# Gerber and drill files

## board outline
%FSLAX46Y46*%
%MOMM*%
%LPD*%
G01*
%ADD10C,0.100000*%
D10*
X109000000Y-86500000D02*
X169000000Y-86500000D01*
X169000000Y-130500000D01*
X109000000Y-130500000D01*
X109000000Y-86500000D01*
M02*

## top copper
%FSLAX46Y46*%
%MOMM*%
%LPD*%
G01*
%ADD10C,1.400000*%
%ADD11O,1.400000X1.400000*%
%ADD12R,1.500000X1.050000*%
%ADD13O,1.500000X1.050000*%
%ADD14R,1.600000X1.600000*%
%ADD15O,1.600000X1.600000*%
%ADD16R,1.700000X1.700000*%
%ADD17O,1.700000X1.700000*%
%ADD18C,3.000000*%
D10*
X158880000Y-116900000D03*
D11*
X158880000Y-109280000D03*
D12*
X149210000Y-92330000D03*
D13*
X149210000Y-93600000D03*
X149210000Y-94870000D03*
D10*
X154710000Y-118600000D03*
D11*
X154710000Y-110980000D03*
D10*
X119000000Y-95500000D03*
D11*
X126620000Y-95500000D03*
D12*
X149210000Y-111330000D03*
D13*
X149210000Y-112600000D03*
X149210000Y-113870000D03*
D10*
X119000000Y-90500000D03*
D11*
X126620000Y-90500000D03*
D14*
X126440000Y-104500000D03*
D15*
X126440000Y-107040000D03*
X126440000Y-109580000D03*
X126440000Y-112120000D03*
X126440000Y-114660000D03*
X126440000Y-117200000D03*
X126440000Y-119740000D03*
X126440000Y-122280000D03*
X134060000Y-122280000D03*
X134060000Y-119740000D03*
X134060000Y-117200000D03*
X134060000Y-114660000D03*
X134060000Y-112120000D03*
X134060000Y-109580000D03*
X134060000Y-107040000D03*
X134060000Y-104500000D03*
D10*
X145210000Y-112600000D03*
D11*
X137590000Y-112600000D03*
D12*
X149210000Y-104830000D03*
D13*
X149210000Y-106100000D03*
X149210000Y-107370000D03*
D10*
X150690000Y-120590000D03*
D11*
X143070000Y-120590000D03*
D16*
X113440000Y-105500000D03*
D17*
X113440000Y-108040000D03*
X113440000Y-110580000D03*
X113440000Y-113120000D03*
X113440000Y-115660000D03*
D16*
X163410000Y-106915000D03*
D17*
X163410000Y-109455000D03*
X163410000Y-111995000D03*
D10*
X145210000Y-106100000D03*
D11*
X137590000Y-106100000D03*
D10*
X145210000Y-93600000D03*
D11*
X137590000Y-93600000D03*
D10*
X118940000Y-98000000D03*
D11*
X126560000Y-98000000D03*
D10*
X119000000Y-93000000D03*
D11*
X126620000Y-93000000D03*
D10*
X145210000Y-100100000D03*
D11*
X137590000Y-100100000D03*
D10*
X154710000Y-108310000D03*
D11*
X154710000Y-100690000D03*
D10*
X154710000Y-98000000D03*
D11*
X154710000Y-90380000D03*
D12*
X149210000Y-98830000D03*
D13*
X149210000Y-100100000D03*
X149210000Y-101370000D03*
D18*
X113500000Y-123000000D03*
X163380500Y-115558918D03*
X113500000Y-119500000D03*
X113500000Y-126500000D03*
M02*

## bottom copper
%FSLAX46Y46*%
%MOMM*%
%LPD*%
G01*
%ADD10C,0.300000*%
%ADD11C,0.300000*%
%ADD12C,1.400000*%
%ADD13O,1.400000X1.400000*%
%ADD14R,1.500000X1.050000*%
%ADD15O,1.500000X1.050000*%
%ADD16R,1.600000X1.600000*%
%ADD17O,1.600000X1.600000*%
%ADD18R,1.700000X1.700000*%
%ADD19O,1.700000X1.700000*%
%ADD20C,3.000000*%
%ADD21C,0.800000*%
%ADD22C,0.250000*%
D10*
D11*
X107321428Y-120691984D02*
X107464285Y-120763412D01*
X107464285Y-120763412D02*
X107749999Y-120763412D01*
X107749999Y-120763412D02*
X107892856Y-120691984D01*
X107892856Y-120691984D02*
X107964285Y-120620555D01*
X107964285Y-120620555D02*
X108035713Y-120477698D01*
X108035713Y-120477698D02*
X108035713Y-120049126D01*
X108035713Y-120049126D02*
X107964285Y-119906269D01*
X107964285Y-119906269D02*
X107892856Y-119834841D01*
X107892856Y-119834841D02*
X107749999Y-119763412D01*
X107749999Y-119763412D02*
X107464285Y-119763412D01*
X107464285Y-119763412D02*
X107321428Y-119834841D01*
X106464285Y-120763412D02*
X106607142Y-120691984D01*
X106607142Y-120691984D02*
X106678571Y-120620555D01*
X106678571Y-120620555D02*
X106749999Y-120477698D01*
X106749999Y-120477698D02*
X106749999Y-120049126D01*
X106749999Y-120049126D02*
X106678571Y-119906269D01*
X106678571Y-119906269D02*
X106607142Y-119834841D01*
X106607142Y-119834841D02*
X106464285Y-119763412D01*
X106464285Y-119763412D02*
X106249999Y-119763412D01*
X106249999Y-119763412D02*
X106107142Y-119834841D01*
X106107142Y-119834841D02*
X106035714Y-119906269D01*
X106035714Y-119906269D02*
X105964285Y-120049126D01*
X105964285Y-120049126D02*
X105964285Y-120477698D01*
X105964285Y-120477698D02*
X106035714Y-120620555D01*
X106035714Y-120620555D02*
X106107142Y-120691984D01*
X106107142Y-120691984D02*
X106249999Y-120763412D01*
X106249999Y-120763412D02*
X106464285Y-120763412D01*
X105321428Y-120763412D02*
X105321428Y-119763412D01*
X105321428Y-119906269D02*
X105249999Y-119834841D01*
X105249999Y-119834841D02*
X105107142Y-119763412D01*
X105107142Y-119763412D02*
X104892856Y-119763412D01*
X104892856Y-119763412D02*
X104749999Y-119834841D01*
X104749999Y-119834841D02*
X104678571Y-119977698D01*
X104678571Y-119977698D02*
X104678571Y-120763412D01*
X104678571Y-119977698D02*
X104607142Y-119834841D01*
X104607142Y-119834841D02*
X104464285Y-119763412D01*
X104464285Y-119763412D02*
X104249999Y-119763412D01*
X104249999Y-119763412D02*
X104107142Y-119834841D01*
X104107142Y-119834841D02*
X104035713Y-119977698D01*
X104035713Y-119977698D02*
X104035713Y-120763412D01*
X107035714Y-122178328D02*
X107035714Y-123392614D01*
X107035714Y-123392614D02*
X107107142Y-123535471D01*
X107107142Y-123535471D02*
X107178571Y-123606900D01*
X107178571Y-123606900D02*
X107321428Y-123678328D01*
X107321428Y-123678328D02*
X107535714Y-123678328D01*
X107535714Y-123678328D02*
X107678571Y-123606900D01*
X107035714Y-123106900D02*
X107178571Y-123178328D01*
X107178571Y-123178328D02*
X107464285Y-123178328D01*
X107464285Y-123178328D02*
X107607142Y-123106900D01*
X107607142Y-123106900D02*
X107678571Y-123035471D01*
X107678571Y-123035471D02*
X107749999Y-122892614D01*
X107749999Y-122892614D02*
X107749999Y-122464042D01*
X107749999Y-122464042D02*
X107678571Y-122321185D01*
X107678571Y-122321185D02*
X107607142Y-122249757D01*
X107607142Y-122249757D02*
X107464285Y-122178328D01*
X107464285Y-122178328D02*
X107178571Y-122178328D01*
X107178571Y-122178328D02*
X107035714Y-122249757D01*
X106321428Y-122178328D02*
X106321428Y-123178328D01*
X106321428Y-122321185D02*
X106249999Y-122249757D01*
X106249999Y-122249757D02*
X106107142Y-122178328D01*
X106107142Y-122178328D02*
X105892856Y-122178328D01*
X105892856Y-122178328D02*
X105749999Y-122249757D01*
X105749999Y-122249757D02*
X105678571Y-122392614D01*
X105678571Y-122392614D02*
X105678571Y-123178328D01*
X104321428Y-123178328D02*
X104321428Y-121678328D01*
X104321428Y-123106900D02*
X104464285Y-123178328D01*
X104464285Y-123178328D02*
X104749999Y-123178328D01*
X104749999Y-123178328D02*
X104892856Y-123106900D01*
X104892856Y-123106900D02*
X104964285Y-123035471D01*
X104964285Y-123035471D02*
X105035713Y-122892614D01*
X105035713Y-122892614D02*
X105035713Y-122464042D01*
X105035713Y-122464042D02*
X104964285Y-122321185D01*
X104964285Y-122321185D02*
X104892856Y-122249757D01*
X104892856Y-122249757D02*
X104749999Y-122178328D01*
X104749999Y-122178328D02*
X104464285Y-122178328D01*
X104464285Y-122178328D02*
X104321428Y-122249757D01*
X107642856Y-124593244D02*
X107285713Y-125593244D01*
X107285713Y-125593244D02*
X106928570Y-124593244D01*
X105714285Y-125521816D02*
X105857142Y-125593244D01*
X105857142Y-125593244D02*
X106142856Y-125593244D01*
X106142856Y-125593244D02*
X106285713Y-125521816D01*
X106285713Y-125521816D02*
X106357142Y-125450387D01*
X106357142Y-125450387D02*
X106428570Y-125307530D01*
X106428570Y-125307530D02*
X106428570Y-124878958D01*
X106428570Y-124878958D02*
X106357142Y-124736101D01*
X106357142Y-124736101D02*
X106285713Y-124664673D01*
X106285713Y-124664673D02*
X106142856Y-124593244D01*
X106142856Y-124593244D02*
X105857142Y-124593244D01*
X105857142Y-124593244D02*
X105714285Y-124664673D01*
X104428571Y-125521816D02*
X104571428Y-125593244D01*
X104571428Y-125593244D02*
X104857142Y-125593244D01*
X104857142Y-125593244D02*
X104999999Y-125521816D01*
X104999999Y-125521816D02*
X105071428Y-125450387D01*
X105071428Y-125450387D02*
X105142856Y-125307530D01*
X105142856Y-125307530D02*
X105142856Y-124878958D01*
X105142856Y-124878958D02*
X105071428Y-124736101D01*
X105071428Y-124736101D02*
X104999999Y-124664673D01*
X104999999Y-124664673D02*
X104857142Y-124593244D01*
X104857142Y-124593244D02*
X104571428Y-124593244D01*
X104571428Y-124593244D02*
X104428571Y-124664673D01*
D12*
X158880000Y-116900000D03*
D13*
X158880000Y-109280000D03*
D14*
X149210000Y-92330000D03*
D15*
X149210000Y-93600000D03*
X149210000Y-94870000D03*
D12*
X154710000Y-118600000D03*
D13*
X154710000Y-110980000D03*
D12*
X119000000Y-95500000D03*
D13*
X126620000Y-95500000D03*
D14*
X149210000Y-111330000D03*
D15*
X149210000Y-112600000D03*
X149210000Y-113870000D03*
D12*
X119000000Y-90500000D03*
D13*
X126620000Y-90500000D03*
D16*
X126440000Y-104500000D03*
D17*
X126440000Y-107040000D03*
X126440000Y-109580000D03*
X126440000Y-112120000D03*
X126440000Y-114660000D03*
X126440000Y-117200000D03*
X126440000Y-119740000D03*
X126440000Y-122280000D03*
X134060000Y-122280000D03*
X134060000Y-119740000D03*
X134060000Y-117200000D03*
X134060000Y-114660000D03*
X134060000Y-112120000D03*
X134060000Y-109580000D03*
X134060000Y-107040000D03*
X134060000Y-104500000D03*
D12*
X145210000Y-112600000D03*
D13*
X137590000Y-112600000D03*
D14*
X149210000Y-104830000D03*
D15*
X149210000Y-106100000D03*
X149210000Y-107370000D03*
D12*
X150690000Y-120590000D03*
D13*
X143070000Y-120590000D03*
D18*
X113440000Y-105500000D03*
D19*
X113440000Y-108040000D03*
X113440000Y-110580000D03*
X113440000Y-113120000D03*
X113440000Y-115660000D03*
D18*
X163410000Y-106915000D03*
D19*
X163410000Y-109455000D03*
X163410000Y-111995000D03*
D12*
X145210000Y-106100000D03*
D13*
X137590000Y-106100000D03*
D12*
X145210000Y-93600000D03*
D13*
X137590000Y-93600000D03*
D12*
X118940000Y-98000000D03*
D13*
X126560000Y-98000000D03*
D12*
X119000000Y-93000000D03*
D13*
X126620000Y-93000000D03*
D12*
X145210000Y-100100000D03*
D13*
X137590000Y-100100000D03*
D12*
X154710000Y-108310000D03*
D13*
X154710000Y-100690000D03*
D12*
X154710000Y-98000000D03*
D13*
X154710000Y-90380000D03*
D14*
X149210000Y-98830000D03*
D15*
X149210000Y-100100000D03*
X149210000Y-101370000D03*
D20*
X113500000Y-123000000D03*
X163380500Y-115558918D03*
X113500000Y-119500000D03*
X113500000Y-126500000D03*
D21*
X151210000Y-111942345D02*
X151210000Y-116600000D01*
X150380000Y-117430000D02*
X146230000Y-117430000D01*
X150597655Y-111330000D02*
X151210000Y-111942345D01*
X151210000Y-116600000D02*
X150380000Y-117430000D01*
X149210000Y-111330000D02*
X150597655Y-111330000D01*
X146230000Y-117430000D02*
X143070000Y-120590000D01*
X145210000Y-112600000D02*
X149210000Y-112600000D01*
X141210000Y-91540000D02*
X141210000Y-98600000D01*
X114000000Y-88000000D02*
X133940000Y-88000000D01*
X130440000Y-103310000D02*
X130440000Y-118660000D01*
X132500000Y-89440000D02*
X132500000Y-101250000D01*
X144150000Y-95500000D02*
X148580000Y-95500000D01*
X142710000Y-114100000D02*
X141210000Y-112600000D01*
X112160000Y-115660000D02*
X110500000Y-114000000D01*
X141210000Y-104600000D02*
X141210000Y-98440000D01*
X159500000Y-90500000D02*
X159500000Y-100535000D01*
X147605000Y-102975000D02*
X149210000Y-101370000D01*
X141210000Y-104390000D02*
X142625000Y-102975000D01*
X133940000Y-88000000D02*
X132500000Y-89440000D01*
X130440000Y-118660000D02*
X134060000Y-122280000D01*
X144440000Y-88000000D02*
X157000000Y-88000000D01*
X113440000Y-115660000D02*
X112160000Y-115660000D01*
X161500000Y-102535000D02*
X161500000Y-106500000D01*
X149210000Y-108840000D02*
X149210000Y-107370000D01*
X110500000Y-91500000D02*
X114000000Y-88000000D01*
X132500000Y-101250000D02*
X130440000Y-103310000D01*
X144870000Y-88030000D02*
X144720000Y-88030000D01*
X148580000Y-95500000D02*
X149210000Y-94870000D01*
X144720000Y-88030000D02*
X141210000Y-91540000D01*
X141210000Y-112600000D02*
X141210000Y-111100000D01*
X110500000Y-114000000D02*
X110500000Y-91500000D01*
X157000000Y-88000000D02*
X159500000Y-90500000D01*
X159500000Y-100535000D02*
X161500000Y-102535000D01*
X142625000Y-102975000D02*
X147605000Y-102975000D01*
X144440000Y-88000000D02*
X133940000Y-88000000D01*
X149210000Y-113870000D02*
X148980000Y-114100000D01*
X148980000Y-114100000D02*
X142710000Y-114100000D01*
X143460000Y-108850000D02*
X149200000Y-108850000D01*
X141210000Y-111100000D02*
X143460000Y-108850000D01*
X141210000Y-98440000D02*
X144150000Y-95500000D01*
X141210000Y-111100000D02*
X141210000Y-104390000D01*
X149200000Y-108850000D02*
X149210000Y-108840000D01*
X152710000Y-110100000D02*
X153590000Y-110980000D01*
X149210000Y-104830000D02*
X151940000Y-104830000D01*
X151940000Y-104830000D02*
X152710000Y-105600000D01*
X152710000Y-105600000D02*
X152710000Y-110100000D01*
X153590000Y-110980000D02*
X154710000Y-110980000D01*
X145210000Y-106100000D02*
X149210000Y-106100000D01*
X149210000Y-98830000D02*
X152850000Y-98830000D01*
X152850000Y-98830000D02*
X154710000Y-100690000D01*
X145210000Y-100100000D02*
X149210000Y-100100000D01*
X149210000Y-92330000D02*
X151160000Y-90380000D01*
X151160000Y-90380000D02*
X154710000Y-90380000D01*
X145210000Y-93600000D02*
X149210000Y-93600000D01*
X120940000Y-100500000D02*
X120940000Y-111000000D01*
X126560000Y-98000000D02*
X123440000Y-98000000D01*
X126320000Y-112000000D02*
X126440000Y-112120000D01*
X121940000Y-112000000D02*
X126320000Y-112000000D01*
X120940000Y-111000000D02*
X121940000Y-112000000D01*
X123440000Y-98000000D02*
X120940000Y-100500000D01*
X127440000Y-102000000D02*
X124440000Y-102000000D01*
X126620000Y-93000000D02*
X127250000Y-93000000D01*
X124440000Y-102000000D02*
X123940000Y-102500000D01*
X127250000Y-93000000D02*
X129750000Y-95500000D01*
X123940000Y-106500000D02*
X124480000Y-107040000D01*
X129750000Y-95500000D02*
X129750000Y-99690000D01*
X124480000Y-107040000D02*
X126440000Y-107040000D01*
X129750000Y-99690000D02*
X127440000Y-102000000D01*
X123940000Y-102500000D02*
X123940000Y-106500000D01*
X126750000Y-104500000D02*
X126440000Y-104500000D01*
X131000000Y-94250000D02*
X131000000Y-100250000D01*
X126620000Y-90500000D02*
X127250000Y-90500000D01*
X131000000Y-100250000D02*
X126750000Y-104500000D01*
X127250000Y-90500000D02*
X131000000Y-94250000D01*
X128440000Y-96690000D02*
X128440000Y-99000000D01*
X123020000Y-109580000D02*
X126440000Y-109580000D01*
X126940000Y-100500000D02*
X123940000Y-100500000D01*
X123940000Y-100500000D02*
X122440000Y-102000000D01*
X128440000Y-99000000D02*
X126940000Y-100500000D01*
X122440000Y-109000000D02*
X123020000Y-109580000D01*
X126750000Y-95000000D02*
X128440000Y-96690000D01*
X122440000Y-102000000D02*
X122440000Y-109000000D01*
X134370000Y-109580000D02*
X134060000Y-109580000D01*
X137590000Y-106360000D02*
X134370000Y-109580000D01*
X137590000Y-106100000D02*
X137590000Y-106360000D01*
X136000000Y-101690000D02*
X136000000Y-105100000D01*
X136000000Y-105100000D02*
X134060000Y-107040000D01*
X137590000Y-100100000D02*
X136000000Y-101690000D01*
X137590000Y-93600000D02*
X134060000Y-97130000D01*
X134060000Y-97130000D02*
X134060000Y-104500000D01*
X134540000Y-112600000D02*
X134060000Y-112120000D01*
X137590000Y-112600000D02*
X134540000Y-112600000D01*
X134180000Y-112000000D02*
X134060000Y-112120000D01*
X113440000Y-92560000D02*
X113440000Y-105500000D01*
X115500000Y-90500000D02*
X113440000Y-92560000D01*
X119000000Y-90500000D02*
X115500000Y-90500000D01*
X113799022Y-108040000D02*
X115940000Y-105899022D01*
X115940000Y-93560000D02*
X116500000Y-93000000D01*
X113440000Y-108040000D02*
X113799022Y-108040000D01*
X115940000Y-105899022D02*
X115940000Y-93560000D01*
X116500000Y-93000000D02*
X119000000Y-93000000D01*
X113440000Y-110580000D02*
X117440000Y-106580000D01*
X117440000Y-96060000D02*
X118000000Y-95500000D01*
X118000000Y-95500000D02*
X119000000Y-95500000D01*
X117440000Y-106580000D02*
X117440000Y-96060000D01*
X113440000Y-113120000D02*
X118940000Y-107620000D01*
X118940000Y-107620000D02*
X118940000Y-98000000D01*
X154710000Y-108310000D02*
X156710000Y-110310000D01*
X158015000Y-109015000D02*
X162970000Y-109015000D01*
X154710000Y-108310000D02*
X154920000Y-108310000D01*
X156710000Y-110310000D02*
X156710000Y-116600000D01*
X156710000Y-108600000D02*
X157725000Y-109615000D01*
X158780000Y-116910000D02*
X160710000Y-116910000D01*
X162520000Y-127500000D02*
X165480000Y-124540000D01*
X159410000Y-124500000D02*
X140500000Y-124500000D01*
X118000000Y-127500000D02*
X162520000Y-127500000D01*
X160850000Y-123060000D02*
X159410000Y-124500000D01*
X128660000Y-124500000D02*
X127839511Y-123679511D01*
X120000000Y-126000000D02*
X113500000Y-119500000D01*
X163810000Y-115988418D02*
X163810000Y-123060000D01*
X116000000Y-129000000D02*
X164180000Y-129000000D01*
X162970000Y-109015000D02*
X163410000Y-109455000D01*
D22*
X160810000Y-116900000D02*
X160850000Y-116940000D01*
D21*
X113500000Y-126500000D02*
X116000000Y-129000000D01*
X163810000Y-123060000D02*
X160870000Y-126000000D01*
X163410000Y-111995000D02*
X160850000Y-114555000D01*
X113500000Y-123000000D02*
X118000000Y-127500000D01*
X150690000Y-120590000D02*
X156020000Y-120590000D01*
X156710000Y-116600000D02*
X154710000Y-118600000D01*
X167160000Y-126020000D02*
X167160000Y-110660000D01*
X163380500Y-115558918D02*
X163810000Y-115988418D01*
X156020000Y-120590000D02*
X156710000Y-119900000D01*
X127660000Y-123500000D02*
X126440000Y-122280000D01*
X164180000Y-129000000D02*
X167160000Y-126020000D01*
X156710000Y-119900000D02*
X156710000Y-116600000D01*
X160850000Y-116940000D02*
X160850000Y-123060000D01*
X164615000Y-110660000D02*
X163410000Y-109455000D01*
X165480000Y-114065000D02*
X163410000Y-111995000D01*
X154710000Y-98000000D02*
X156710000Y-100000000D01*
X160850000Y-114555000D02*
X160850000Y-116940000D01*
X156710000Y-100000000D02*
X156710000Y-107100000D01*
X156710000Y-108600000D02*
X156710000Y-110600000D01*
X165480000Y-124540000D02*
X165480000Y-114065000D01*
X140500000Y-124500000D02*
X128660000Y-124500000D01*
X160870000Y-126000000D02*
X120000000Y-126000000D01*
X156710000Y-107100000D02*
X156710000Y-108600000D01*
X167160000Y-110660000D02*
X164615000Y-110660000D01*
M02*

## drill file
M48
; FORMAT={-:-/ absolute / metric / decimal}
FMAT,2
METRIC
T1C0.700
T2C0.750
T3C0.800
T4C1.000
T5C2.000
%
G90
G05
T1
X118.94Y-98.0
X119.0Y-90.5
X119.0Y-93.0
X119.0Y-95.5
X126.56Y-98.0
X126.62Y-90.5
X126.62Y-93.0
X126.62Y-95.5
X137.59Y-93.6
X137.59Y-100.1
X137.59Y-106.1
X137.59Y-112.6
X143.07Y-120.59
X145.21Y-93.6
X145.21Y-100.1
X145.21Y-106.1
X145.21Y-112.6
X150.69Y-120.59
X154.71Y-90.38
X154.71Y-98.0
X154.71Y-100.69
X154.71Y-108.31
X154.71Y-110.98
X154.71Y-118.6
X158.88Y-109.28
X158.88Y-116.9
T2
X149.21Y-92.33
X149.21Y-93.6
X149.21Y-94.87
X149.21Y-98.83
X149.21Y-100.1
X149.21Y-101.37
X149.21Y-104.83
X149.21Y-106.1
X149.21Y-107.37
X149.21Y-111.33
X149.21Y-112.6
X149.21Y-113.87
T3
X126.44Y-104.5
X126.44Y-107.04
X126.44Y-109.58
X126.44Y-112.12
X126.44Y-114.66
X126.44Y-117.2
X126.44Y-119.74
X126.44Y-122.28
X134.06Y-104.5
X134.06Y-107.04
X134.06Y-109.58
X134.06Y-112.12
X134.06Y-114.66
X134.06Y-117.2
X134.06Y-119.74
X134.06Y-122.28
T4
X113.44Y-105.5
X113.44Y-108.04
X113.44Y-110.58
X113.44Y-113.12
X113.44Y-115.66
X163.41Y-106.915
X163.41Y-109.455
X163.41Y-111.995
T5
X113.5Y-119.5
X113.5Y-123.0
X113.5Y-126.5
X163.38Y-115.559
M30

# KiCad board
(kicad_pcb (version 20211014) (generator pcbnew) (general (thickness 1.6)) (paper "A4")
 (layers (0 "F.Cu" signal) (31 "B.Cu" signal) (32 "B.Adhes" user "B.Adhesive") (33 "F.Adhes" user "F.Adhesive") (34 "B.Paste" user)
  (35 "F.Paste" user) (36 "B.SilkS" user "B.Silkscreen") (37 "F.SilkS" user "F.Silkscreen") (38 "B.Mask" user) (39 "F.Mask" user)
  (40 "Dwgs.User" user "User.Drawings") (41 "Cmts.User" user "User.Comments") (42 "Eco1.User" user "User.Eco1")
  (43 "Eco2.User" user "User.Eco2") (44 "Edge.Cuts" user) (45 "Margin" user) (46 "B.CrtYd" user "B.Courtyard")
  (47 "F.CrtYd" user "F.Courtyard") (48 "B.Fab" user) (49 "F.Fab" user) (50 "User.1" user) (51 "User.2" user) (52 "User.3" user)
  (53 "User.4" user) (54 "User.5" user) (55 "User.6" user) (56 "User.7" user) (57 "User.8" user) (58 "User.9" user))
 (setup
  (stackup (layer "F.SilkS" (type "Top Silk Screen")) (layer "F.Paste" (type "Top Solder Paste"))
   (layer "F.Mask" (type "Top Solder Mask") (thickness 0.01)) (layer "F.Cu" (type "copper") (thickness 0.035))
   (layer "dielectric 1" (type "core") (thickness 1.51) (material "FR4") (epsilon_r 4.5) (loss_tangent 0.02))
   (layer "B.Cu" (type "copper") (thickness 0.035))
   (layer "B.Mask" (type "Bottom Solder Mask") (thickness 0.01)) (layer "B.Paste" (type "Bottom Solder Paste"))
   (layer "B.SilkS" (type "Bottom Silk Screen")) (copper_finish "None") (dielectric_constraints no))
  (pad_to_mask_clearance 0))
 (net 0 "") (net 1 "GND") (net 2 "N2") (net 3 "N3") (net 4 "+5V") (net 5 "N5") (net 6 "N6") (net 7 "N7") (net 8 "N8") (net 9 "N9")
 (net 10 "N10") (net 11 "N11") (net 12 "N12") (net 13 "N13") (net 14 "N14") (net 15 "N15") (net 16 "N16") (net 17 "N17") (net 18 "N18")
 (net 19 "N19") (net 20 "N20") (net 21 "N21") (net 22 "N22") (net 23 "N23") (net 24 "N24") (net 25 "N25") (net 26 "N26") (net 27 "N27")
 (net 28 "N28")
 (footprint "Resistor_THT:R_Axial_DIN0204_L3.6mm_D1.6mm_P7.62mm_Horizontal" (layer "F.Cu") (at 158.88 116.9 90)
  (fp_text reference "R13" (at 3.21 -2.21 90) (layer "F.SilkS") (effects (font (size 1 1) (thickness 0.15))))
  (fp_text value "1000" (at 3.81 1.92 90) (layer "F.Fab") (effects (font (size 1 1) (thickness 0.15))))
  (pad "1" thru_hole circle (at 0 0 90) (size 1.4 1.4) (drill 0.7) (layers *.Cu *.Mask) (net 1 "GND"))
  (pad "2" thru_hole oval (at 7.62 0 90) (size 1.4 1.4) (drill 0.7) (layers *.Cu *.Mask) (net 1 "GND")))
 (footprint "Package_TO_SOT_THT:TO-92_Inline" (layer "F.Cu") (at 149.21 92.33 -90)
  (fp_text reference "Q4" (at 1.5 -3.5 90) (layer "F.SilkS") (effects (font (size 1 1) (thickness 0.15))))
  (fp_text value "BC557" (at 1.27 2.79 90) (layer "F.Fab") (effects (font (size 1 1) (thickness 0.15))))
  (pad "1" thru_hole rect (at 0 0 270) (size 1.05 1.5) (drill 0.75) (layers *.Cu *.Mask) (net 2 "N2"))
  (pad "2" thru_hole oval (at 1.27 0 270) (size 1.05 1.5) (drill 0.75) (layers *.Cu *.Mask) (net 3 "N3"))
  (pad "3" thru_hole oval (at 2.54 0 270) (size 1.05 1.5) (drill 0.75) (layers *.Cu *.Mask) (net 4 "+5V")))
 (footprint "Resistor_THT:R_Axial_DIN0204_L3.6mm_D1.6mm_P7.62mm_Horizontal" (layer "F.Cu") (at 154.71 118.6 90)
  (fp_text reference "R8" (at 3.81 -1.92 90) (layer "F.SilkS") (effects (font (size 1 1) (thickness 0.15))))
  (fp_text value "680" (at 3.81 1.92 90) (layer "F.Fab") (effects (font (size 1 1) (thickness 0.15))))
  (pad "1" thru_hole circle (at 0 0 90) (size 1.4 1.4) (drill 0.7) (layers *.Cu *.Mask) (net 1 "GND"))
  (pad "2" thru_hole oval (at 7.62 0 90) (size 1.4 1.4) (drill 0.7) (layers *.Cu *.Mask) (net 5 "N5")))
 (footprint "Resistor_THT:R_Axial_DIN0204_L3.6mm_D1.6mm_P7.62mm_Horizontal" (layer "F.Cu") (at 119 95.5)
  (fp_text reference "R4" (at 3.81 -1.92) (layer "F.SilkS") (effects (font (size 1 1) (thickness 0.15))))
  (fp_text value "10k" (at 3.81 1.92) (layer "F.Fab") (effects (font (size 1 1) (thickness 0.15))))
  (pad "1" thru_hole circle (at 0 0) (size 1.4 1.4) (drill 0.7) (layers *.Cu *.Mask) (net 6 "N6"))
  (pad "2" thru_hole oval (at 7.62 0) (size 1.4 1.4) (drill 0.7) (layers *.Cu *.Mask) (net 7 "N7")))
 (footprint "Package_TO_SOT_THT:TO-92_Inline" (layer "F.Cu") (at 149.21 111.33 -90)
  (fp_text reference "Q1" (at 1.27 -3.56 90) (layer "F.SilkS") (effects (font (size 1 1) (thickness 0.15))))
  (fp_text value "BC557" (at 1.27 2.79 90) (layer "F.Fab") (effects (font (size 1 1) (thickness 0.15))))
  (pad "1" thru_hole rect (at 0 0 270) (size 1.05 1.5) (drill 0.75) (layers *.Cu *.Mask) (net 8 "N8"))
  (pad "2" thru_hole oval (at 1.27 0 270) (size 1.05 1.5) (drill 0.75) (layers *.Cu *.Mask) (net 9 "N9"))
  (pad "3" thru_hole oval (at 2.54 0 270) (size 1.05 1.5) (drill 0.75) (layers *.Cu *.Mask) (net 4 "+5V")))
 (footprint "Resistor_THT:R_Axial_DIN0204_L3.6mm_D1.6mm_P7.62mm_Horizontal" (layer "F.Cu") (at 119 90.5)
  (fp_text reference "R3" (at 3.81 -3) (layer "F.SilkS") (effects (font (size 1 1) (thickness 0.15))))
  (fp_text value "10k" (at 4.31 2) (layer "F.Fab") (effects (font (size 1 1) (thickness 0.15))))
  (pad "1" thru_hole circle (at 0 0) (size 1.4 1.4) (drill 0.7) (layers *.Cu *.Mask) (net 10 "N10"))
  (pad "2" thru_hole oval (at 7.62 0) (size 1.4 1.4) (drill 0.7) (layers *.Cu *.Mask) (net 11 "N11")))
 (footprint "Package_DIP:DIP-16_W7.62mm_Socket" (layer "F.Cu") (at 126.44 104.5)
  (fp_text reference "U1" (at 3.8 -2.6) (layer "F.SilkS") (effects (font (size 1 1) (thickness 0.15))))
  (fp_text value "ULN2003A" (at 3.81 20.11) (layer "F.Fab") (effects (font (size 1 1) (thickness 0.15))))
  (pad "1" thru_hole rect (at 0 0) (size 1.6 1.6) (drill 0.8) (layers *.Cu *.Mask) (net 11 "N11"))
  (pad "2" thru_hole oval (at 0 2.54) (size 1.6 1.6) (drill 0.8) (layers *.Cu *.Mask) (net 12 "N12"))
  (pad "3" thru_hole oval (at 0 5.08) (size 1.6 1.6) (drill 0.8) (layers *.Cu *.Mask) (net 7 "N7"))
  (pad "4" thru_hole oval (at 0 7.62) (size 1.6 1.6) (drill 0.8) (layers *.Cu *.Mask) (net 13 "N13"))
  (pad "5" thru_hole oval (at 0 10.16) (size 1.6 1.6) (drill 0.8) (layers *.Cu *.Mask) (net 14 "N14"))
  (pad "6" thru_hole oval (at 0 12.7) (size 1.6 1.6) (drill 0.8) (layers *.Cu *.Mask) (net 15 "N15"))
  (pad "7" thru_hole oval (at 0 15.24) (size 1.6 1.6) (drill 0.8) (layers *.Cu *.Mask) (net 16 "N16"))
  (pad "8" thru_hole oval (at 0 17.78) (size 1.6 1.6) (drill 0.8) (layers *.Cu *.Mask) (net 1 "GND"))
  (pad "9" thru_hole oval (at 7.62 17.78) (size 1.6 1.6) (drill 0.8) (layers *.Cu *.Mask) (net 4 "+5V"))
  (pad "10" thru_hole oval (at 7.62 15.24) (size 1.6 1.6) (drill 0.8) (layers *.Cu *.Mask) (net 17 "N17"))
  (pad "11" thru_hole oval (at 7.62 12.7) (size 1.6 1.6) (drill 0.8) (layers *.Cu *.Mask) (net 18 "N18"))
  (pad "12" thru_hole oval (at 7.62 10.16) (size 1.6 1.6) (drill 0.8) (layers *.Cu *.Mask) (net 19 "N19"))
  (pad "13" thru_hole oval (at 7.62 7.62) (size 1.6 1.6) (drill 0.8) (layers *.Cu *.Mask) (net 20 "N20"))
  (pad "14" thru_hole oval (at 7.62 5.08) (size 1.6 1.6) (drill 0.8) (layers *.Cu *.Mask) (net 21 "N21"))
  (pad "15" thru_hole oval (at 7.62 2.54) (size 1.6 1.6) (drill 0.8) (layers *.Cu *.Mask) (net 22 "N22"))
  (pad "16" thru_hole oval (at 7.62 0) (size 1.6 1.6) (drill 0.8) (layers *.Cu *.Mask) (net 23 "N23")))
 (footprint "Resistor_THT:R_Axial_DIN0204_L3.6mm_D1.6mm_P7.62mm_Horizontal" (layer "F.Cu") (at 145.21 112.6 180)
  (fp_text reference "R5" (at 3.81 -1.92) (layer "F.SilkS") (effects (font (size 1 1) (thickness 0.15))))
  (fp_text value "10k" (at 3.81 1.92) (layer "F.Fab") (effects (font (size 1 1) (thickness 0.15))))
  (pad "1" thru_hole circle (at 0 0 180) (size 1.4 1.4) (drill 0.7) (layers *.Cu *.Mask) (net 9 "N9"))
  (pad "2" thru_hole oval (at 7.62 0 180) (size 1.4 1.4) (drill 0.7) (layers *.Cu *.Mask) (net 20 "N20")))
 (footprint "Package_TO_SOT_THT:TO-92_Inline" (layer "F.Cu") (at 149.21 104.83 -90)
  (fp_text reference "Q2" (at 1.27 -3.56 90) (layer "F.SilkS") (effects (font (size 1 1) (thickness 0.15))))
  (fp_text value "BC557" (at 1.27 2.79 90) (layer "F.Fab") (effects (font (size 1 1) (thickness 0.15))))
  (pad "1" thru_hole rect (at 0 0 270) (size 1.05 1.5) (drill 0.75) (layers *.Cu *.Mask) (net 5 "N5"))
  (pad "2" thru_hole oval (at 1.27 0 270) (size 1.05 1.5) (drill 0.75) (layers *.Cu *.Mask) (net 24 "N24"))
  (pad "3" thru_hole oval (at 2.54 0 270) (size 1.05 1.5) (drill 0.75) (layers *.Cu *.Mask) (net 4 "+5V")))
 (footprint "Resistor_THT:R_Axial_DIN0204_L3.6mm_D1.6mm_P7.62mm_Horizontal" (layer "F.Cu") (at 150.69 120.59 180)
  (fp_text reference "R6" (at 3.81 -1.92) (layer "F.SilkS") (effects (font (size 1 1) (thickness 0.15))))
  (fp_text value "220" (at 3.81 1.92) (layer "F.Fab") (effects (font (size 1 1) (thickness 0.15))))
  (pad "1" thru_hole circle (at 0 0 180) (size 1.4 1.4) (drill 0.7) (layers *.Cu *.Mask) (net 1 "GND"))
  (pad "2" thru_hole oval (at 7.62 0 180) (size 1.4 1.4) (drill 0.7) (layers *.Cu *.Mask) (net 8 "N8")))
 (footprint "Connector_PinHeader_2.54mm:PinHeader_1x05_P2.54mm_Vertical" (layer "F.Cu") (at 113.44 105.5)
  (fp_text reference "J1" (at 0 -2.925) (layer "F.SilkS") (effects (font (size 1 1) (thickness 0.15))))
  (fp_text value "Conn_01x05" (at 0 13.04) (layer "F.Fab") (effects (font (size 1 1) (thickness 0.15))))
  (pad "1" thru_hole rect (at 0 0) (size 1.7 1.7) (drill 1) (layers *.Cu *.Mask) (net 10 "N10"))
  (pad "2" thru_hole oval (at 0 2.54) (size 1.7 1.7) (drill 1) (layers *.Cu *.Mask) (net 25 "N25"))
  (pad "3" thru_hole oval (at 0 5.08) (size 1.7 1.7) (drill 1) (layers *.Cu *.Mask) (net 6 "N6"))
  (pad "4" thru_hole oval (at 0 7.62) (size 1.7 1.7) (drill 1) (layers *.Cu *.Mask) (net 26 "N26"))
  (pad "5" thru_hole oval (at 0 10.16) (size 1.7 1.7) (drill 1) (layers *.Cu *.Mask) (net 4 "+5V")))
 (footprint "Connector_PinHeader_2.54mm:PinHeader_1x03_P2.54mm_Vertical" (layer "F.Cu") (at 163.41 106.915)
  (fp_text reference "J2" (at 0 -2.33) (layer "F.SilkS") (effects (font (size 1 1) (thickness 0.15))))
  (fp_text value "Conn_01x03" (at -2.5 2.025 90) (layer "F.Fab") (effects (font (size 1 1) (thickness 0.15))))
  (pad "1" thru_hole rect (at 0 0) (size 1.7 1.7) (drill 1) (layers *.Cu *.Mask) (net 4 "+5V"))
  (pad "2" thru_hole oval (at 0 2.54) (size 1.7 1.7) (drill 1) (layers *.Cu *.Mask) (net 1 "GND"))
  (pad "3" thru_hole oval (at 0 5.08) (size 1.7 1.7) (drill 1) (layers *.Cu *.Mask) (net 1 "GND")))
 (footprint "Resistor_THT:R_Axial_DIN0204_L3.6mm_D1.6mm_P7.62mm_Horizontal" (layer "F.Cu") (at 145.21 106.1 180)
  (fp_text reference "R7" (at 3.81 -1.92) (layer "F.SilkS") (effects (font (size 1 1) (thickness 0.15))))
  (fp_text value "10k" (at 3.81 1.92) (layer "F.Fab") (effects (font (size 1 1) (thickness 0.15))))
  (pad "1" thru_hole circle (at 0 0 180) (size 1.4 1.4) (drill 0.7) (layers *.Cu *.Mask) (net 24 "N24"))
  (pad "2" thru_hole oval (at 7.62 0 180) (size 1.4 1.4) (drill 0.7) (layers *.Cu *.Mask) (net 21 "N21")))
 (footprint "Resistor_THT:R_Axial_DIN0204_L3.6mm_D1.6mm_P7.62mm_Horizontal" (layer "F.Cu") (at 145.21 93.6 180)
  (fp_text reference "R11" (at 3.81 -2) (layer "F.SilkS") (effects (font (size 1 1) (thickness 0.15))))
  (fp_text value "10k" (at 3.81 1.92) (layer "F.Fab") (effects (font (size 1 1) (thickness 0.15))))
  (pad "1" thru_hole circle (at 0 0 180) (size 1.4 1.4) (drill 0.7) (layers *.Cu *.Mask) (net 3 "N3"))
  (pad "2" thru_hole oval (at 7.62 0 180) (size 1.4 1.4) (drill 0.7) (layers *.Cu *.Mask) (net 23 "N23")))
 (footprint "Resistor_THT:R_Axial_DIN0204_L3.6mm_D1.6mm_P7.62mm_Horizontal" (layer "F.Cu") (at 118.94 98)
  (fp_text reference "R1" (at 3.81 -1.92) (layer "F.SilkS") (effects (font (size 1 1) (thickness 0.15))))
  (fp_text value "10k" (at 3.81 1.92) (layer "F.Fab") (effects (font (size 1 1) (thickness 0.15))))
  (pad "1" thru_hole circle (at 0 0) (size 1.4 1.4) (drill 0.7) (layers *.Cu *.Mask) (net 26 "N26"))
  (pad "2" thru_hole oval (at 7.62 0) (size 1.4 1.4) (drill 0.7) (layers *.Cu *.Mask) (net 13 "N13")))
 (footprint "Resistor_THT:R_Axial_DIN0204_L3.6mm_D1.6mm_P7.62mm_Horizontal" (layer "F.Cu") (at 119 93)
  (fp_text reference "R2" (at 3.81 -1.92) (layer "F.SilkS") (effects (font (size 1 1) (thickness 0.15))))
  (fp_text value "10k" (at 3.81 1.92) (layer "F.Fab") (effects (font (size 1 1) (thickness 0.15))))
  (pad "1" thru_hole circle (at 0 0) (size 1.4 1.4) (drill 0.7) (layers *.Cu *.Mask) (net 25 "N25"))
  (pad "2" thru_hole oval (at 7.62 0) (size 1.4 1.4) (drill 0.7) (layers *.Cu *.Mask) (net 12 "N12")))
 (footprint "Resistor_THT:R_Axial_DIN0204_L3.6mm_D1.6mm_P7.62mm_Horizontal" (layer "F.Cu") (at 145.21 100.1 180)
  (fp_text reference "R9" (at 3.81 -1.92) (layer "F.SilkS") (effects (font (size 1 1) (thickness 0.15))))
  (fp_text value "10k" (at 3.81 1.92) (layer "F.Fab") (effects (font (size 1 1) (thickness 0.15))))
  (pad "1" thru_hole circle (at 0 0 180) (size 1.4 1.4) (drill 0.7) (layers *.Cu *.Mask) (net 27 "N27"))
  (pad "2" thru_hole oval (at 7.62 0 180) (size 1.4 1.4) (drill 0.7) (layers *.Cu *.Mask) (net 22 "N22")))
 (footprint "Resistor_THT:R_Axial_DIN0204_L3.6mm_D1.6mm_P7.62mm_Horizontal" (layer "F.Cu") (at 154.71 108.31 90)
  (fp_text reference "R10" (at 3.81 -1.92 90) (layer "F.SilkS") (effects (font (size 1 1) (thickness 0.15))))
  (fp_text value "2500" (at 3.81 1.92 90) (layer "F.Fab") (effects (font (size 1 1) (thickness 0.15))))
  (pad "1" thru_hole circle (at 0 0 90) (size 1.4 1.4) (drill 0.7) (layers *.Cu *.Mask) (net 1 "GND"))
  (pad "2" thru_hole oval (at 7.62 0 90) (size 1.4 1.4) (drill 0.7) (layers *.Cu *.Mask) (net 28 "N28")))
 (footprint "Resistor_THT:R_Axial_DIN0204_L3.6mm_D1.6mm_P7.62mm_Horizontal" (layer "F.Cu") (at 154.71 98 90)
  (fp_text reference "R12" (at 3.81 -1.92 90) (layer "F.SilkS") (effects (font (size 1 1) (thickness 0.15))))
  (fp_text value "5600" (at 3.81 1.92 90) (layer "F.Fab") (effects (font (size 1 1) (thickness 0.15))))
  (pad "1" thru_hole circle (at 0 0 90) (size 1.4 1.4) (drill 0.7) (layers *.Cu *.Mask) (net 1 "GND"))
  (pad "2" thru_hole oval (at 7.62 0 90) (size 1.4 1.4) (drill 0.7) (layers *.Cu *.Mask) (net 2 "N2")))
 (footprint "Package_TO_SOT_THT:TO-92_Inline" (layer "F.Cu") (at 149.21 98.83 -90)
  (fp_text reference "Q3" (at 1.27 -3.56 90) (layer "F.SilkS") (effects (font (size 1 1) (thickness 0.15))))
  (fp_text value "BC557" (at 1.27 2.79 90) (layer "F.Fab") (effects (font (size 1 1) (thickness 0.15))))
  (pad "1" thru_hole rect (at 0 0 270) (size 1.05 1.5) (drill 0.75) (layers *.Cu *.Mask) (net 28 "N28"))
  (pad "2" thru_hole oval (at 1.27 0 270) (size 1.05 1.5) (drill 0.75) (layers *.Cu *.Mask) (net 27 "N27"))
  (pad "3" thru_hole oval (at 2.54 0 270) (size 1.05 1.5) (drill 0.75) (layers *.Cu *.Mask) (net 4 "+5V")))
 (gr_rect (start 169 130.5) (end 109 86.5) (layer "Edge.Cuts") (width 0.1) (fill none))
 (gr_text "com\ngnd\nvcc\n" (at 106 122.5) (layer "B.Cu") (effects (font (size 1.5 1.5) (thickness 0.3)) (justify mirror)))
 (via (at 113.5 123) (size 3) (drill 2) (layers "F.Cu" "B.Cu") (free) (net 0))
 (via (at 163.3805 115.558918) (size 3) (drill 2) (layers "F.Cu" "B.Cu") (free) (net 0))
 (via (at 113.5 119.5) (size 3) (drill 2) (layers "F.Cu" "B.Cu") (free) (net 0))
 (via (at 113.5 126.5) (size 3) (drill 2) (layers "F.Cu" "B.Cu") (free) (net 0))
 (segment (start 151.21 111.942345) (end 151.21 116.6) (width 0.8) (layer "B.Cu") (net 8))
 (segment (start 150.38 117.43) (end 146.23 117.43) (width 0.8) (layer "B.Cu") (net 8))
 (segment (start 150.597655 111.33) (end 151.21 111.942345) (width 0.8) (layer "B.Cu") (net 8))
 (segment (start 151.21 116.6) (end 150.38 117.43) (width 0.8) (layer "B.Cu") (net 8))
 (segment (start 149.21 111.33) (end 150.597655 111.33) (width 0.8) (layer "B.Cu") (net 8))
 (segment (start 146.23 117.43) (end 143.07 120.59) (width 0.8) (layer "B.Cu") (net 8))
 (segment (start 145.21 112.6) (end 149.21 112.6) (width 0.8) (layer "B.Cu") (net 9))
 (segment (start 141.21 91.54) (end 141.21 98.6) (width 0.8) (layer "B.Cu") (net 4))
 (segment (start 114 88) (end 133.94 88) (width 0.8) (layer "B.Cu") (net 4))
 (segment (start 130.44 103.31) (end 130.44 118.66) (width 0.8) (layer "B.Cu") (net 4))
 (segment (start 132.5 89.44) (end 132.5 101.25) (width 0.8) (layer "B.Cu") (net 4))
 (segment (start 144.15 95.5) (end 148.58 95.5) (width 0.8) (layer "B.Cu") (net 4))
 (segment (start 142.71 114.1) (end 141.21 112.6) (width 0.8) (layer "B.Cu") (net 4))
 (segment (start 112.16 115.66) (end 110.5 114) (width 0.8) (layer "B.Cu") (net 4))
 (segment (start 141.21 104.6) (end 141.21 98.44) (width 0.8) (layer "B.Cu") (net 4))
 (segment (start 159.5 90.5) (end 159.5 100.535) (width 0.8) (layer "B.Cu") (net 4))
 (segment (start 147.605 102.975) (end 149.21 101.37) (width 0.8) (layer "B.Cu") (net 4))
 (segment (start 141.21 104.39) (end 142.625 102.975) (width 0.8) (layer "B.Cu") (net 4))
 (segment (start 133.94 88) (end 132.5 89.44) (width 0.8) (layer "B.Cu") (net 4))
 (segment (start 130.44 118.66) (end 134.06 122.28) (width 0.8) (layer "B.Cu") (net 4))
 (segment (start 144.44 88) (end 157 88) (width 0.8) (layer "B.Cu") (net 4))
 (segment (start 113.44 115.66) (end 112.16 115.66) (width 0.8) (layer "B.Cu") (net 4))
 (segment (start 161.5 102.535) (end 161.5 106.5) (width 0.8) (layer "B.Cu") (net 4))
 (segment (start 149.21 108.84) (end 149.21 107.37) (width 0.8) (layer "B.Cu") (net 4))
 (segment (start 110.5 91.5) (end 114 88) (width 0.8) (layer "B.Cu") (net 4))
 (segment (start 132.5 101.25) (end 130.44 103.31) (width 0.8) (layer "B.Cu") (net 4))
 (segment (start 144.87 88.03) (end 144.72 88.03) (width 0.8) (layer "B.Cu") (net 4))
 (segment (start 148.58 95.5) (end 149.21 94.87) (width 0.8) (layer "B.Cu") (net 4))
 (segment (start 144.72 88.03) (end 141.21 91.54) (width 0.8) (layer "B.Cu") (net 4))
 (segment (start 141.21 112.6) (end 141.21 111.1) (width 0.8) (layer "B.Cu") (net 4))
 (segment (start 110.5 114) (end 110.5 91.5) (width 0.8) (layer "B.Cu") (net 4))
 (segment (start 157 88) (end 159.5 90.5) (width 0.8) (layer "B.Cu") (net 4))
 (segment (start 159.5 100.535) (end 161.5 102.535) (width 0.8) (layer "B.Cu") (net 4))
 (segment (start 142.625 102.975) (end 147.605 102.975) (width 0.8) (layer "B.Cu") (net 4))
 (segment (start 144.44 88) (end 133.94 88) (width 0.8) (layer "B.Cu") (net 4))
 (segment (start 149.21 113.87) (end 148.98 114.1) (width 0.8) (layer "B.Cu") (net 4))
 (segment (start 148.98 114.1) (end 142.71 114.1) (width 0.8) (layer "B.Cu") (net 4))
 (segment (start 143.46 108.85) (end 149.2 108.85) (width 0.8) (layer "B.Cu") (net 4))
 (segment (start 141.21 111.1) (end 143.46 108.85) (width 0.8) (layer "B.Cu") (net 4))
 (segment (start 141.21 98.44) (end 144.15 95.5) (width 0.8) (layer "B.Cu") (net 4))
 (segment (start 141.21 111.1) (end 141.21 104.39) (width 0.8) (layer "B.Cu") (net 4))
 (segment (start 149.2 108.85) (end 149.21 108.84) (width 0.8) (layer "B.Cu") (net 4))
 (segment (start 152.71 110.1) (end 153.59 110.98) (width 0.8) (layer "B.Cu") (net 5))
 (segment (start 149.21 104.83) (end 151.94 104.83) (width 0.8) (layer "B.Cu") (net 5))
 (segment (start 151.94 104.83) (end 152.71 105.6) (width 0.8) (layer "B.Cu") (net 5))
 (segment (start 152.71 105.6) (end 152.71 110.1) (width 0.8) (layer "B.Cu") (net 5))
 (segment (start 153.59 110.98) (end 154.71 110.98) (width 0.8) (layer "B.Cu") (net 5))
 (segment (start 145.21 106.1) (end 149.21 106.1) (width 0.8) (layer "B.Cu") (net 24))
 (segment (start 149.21 98.83) (end 152.85 98.83) (width 0.8) (layer "B.Cu") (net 28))
 (segment (start 152.85 98.83) (end 154.71 100.69) (width 0.8) (layer "B.Cu") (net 28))
 (segment (start 145.21 100.1) (end 149.21 100.1) (width 0.8) (layer "B.Cu") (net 27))
 (segment (start 149.21 92.33) (end 151.16 90.38) (width 0.8) (layer "B.Cu") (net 2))
 (segment (start 151.16 90.38) (end 154.71 90.38) (width 0.8) (layer "B.Cu") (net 2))
 (segment (start 145.21 93.6) (end 149.21 93.6) (width 0.8) (layer "B.Cu") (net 3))
 (segment (start 120.94 100.5) (end 120.94 111) (width 0.8) (layer "B.Cu") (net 13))
 (segment (start 126.56 98) (end 123.44 98) (width 0.8) (layer "B.Cu") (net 13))
 (segment (start 126.32 112) (end 126.44 112.12) (width 0.8) (layer "B.Cu") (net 13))
 (segment (start 121.94 112) (end 126.32 112) (width 0.8) (layer "B.Cu") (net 13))
 (segment (start 120.94 111) (end 121.94 112) (width 0.8) (layer "B.Cu") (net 13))
 (segment (start 123.44 98) (end 120.94 100.5) (width 0.8) (layer "B.Cu") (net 13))
 (segment (start 127.44 102) (end 124.44 102) (width 0.8) (layer "B.Cu") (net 12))
 (segment (start 126.62 93) (end 127.25 93) (width 0.8) (layer "B.Cu") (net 12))
 (segment (start 124.44 102) (end 123.94 102.5) (width 0.8) (layer "B.Cu") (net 12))
 (segment (start 127.25 93) (end 129.75 95.5) (width 0.8) (layer "B.Cu") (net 12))
 (segment (start 123.94 106.5) (end 124.48 107.04) (width 0.8) (layer "B.Cu") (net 12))
 (segment (start 129.75 95.5) (end 129.75 99.69) (width 0.8) (layer "B.Cu") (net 12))
 (segment (start 124.48 107.04) (end 126.44 107.04) (width 0.8) (layer "B.Cu") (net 12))
 (segment (start 129.75 99.69) (end 127.44 102) (width 0.8) (layer "B.Cu") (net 12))
 (segment (start 123.94 102.5) (end 123.94 106.5) (width 0.8) (layer "B.Cu") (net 12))
 (segment (start 126.75 104.5) (end 126.44 104.5) (width 0.8) (layer "B.Cu") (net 11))
 (segment (start 131 94.25) (end 131 100.25) (width 0.8) (layer "B.Cu") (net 11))
 (segment (start 126.62 90.5) (end 127.25 90.5) (width 0.8) (layer "B.Cu") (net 11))
 (segment (start 131 100.25) (end 126.75 104.5) (width 0.8) (layer "B.Cu") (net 11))
 (segment (start 127.25 90.5) (end 131 94.25) (width 0.8) (layer "B.Cu") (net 11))
 (segment (start 128.44 96.69) (end 128.44 99) (width 0.8) (layer "B.Cu") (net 7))
 (segment (start 123.02 109.58) (end 126.44 109.58) (width 0.8) (layer "B.Cu") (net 7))
 (segment (start 126.94 100.5) (end 123.94 100.5) (width 0.8) (layer "B.Cu") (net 7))
 (segment (start 123.94 100.5) (end 122.44 102) (width 0.8) (layer "B.Cu") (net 7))
 (segment (start 128.44 99) (end 126.94 100.5) (width 0.8) (layer "B.Cu") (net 7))
 (segment (start 122.44 109) (end 123.02 109.58) (width 0.8) (layer "B.Cu") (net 7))
 (segment (start 126.75 95) (end 128.44 96.69) (width 0.8) (layer "B.Cu") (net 7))
 (segment (start 122.44 102) (end 122.44 109) (width 0.8) (layer "B.Cu") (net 7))
 (segment (start 134.37 109.58) (end 134.06 109.58) (width 0.8) (layer "B.Cu") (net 21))
 (segment (start 137.59 106.36) (end 134.37 109.58) (width 0.8) (layer "B.Cu") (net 21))
 (segment (start 137.59 106.1) (end 137.59 106.36) (width 0.8) (layer "B.Cu") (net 21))
 (segment (start 136 101.69) (end 136 105.1) (width 0.8) (layer "B.Cu") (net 22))
 (segment (start 136 105.1) (end 134.06 107.04) (width 0.8) (layer "B.Cu") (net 22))
 (segment (start 137.59 100.1) (end 136 101.69) (width 0.8) (layer "B.Cu") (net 22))
 (segment (start 137.59 93.6) (end 134.06 97.13) (width 0.8) (layer "B.Cu") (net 23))
 (segment (start 134.06 97.13) (end 134.06 104.5) (width 0.8) (layer "B.Cu") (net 23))
 (segment (start 134.54 112.6) (end 134.06 112.12) (width 0.8) (layer "B.Cu") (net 20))
 (segment (start 137.59 112.6) (end 134.54 112.6) (width 0.8) (layer "B.Cu") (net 20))
 (segment (start 134.18 112) (end 134.06 112.12) (width 0.8) (layer "B.Cu") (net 20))
 (segment (start 113.44 92.56) (end 113.44 105.5) (width 0.8) (layer "B.Cu") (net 10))
 (segment (start 115.5 90.5) (end 113.44 92.56) (width 0.8) (layer "B.Cu") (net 10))
 (segment (start 119 90.5) (end 115.5 90.5) (width 0.8) (layer "B.Cu") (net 10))
 (segment (start 113.799022 108.04) (end 115.94 105.899022) (width 0.8) (layer "B.Cu") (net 25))
 (segment (start 115.94 93.56) (end 116.5 93) (width 0.8) (layer "B.Cu") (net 25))
 (segment (start 113.44 108.04) (end 113.799022 108.04) (width 0.8) (layer "B.Cu") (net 25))
 (segment (start 115.94 105.899022) (end 115.94 93.56) (width 0.8) (layer "B.Cu") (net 25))
 (segment (start 116.5 93) (end 119 93) (width 0.8) (layer "B.Cu") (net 25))
 (segment (start 113.44 110.58) (end 117.44 106.58) (width 0.8) (layer "B.Cu") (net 6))
 (segment (start 117.44 96.06) (end 118 95.5) (width 0.8) (layer "B.Cu") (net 6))
 (segment (start 118 95.5) (end 119 95.5) (width 0.8) (layer "B.Cu") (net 6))
 (segment (start 117.44 106.58) (end 117.44 96.06) (width 0.8) (layer "B.Cu") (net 6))
 (segment (start 113.44 113.12) (end 118.94 107.62) (width 0.8) (layer "B.Cu") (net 26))
 (segment (start 118.94 107.62) (end 118.94 98) (width 0.8) (layer "B.Cu") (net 26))
 (segment (start 154.71 108.31) (end 156.71 110.31) (width 0.8) (layer "B.Cu") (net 1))
 (segment (start 158.015 109.015) (end 162.97 109.015) (width 0.8) (layer "B.Cu") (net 1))
 (segment (start 154.71 108.31) (end 154.92 108.31) (width 0.8) (layer "B.Cu") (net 1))
 (segment (start 156.71 110.31) (end 156.71 116.6) (width 0.8) (layer "B.Cu") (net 1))
 (segment (start 156.71 108.6) (end 157.725 109.615) (width 0.8) (layer "B.Cu") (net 1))
 (segment (start 158.78 116.91) (end 160.71 116.91) (width 0.8) (layer "B.Cu") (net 1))
 (segment (start 162.52 127.5) (end 165.48 124.54) (width 0.8) (layer "B.Cu") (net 1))
 (segment (start 159.41 124.5) (end 140.5 124.5) (width 0.8) (layer "B.Cu") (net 1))
 (segment (start 118 127.5) (end 162.52 127.5) (width 0.8) (layer "B.Cu") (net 1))
 (segment (start 160.85 123.06) (end 159.41 124.5) (width 0.8) (layer "B.Cu") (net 1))
 (segment (start 128.66 124.5) (end 127.839511 123.679511) (width 0.8) (layer "B.Cu") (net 1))
 (segment (start 120 126) (end 113.5 119.5) (width 0.8) (layer "B.Cu") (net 1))
 (segment (start 163.81 115.988418) (end 163.81 123.06) (width 0.8) (layer "B.Cu") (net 1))
 (segment (start 116 129) (end 164.18 129) (width 0.8) (layer "B.Cu") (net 1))
 (segment (start 162.97 109.015) (end 163.41 109.455) (width 0.8) (layer "B.Cu") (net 1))
 (segment (start 160.81 116.9) (end 160.85 116.94) (width 0.25) (layer "B.Cu") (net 1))
 (segment (start 113.5 126.5) (end 116 129) (width 0.8) (layer "B.Cu") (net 1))
 (segment (start 163.81 123.06) (end 160.87 126) (width 0.8) (layer "B.Cu") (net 1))
 (segment (start 163.41 111.995) (end 160.85 114.555) (width 0.8) (layer "B.Cu") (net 1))
 (segment (start 113.5 123) (end 118 127.5) (width 0.8) (layer "B.Cu") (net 1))
 (segment (start 150.69 120.59) (end 156.02 120.59) (width 0.8) (layer "B.Cu") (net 1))
 (segment (start 156.71 116.6) (end 154.71 118.6) (width 0.8) (layer "B.Cu") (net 1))
 (segment (start 167.16 126.02) (end 167.16 110.66) (width 0.8) (layer "B.Cu") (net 1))
 (segment (start 163.3805 115.558918) (end 163.81 115.988418) (width 0.8) (layer "B.Cu") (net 1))
 (segment (start 156.02 120.59) (end 156.71 119.9) (width 0.8) (layer "B.Cu") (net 1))
 (segment (start 127.66 123.5) (end 126.44 122.28) (width 0.8) (layer "B.Cu") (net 1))
 (segment (start 164.18 129) (end 167.16 126.02) (width 0.8) (layer "B.Cu") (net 1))
 (segment (start 156.71 119.9) (end 156.71 116.6) (width 0.8) (layer "B.Cu") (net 1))
 (segment (start 160.85 116.94) (end 160.85 123.06) (width 0.8) (layer "B.Cu") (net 1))
 (segment (start 164.615 110.66) (end 163.41 109.455) (width 0.8) (layer "B.Cu") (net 1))
 (segment (start 165.48 114.065) (end 163.41 111.995) (width 0.8) (layer "B.Cu") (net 1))
 (segment (start 154.71 98) (end 156.71 100) (width 0.8) (layer "B.Cu") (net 1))
 (segment (start 160.85 114.555) (end 160.85 116.94) (width 0.8) (layer "B.Cu") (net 1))
 (segment (start 156.71 100) (end 156.71 107.1) (width 0.8) (layer "B.Cu") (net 1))
 (segment (start 156.71 108.6) (end 156.71 110.6) (width 0.8) (layer "B.Cu") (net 1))
 (segment (start 165.48 124.54) (end 165.48 114.065) (width 0.8) (layer "B.Cu") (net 1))
 (segment (start 140.5 124.5) (end 128.66 124.5) (width 0.8) (layer "B.Cu") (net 1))
 (segment (start 160.87 126) (end 120 126) (width 0.8) (layer "B.Cu") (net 1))
 (segment (start 156.71 107.1) (end 156.71 108.6) (width 0.8) (layer "B.Cu") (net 1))
 (segment (start 167.16 110.66) (end 164.615 110.66) (width 0.8) (layer "B.Cu") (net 1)))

